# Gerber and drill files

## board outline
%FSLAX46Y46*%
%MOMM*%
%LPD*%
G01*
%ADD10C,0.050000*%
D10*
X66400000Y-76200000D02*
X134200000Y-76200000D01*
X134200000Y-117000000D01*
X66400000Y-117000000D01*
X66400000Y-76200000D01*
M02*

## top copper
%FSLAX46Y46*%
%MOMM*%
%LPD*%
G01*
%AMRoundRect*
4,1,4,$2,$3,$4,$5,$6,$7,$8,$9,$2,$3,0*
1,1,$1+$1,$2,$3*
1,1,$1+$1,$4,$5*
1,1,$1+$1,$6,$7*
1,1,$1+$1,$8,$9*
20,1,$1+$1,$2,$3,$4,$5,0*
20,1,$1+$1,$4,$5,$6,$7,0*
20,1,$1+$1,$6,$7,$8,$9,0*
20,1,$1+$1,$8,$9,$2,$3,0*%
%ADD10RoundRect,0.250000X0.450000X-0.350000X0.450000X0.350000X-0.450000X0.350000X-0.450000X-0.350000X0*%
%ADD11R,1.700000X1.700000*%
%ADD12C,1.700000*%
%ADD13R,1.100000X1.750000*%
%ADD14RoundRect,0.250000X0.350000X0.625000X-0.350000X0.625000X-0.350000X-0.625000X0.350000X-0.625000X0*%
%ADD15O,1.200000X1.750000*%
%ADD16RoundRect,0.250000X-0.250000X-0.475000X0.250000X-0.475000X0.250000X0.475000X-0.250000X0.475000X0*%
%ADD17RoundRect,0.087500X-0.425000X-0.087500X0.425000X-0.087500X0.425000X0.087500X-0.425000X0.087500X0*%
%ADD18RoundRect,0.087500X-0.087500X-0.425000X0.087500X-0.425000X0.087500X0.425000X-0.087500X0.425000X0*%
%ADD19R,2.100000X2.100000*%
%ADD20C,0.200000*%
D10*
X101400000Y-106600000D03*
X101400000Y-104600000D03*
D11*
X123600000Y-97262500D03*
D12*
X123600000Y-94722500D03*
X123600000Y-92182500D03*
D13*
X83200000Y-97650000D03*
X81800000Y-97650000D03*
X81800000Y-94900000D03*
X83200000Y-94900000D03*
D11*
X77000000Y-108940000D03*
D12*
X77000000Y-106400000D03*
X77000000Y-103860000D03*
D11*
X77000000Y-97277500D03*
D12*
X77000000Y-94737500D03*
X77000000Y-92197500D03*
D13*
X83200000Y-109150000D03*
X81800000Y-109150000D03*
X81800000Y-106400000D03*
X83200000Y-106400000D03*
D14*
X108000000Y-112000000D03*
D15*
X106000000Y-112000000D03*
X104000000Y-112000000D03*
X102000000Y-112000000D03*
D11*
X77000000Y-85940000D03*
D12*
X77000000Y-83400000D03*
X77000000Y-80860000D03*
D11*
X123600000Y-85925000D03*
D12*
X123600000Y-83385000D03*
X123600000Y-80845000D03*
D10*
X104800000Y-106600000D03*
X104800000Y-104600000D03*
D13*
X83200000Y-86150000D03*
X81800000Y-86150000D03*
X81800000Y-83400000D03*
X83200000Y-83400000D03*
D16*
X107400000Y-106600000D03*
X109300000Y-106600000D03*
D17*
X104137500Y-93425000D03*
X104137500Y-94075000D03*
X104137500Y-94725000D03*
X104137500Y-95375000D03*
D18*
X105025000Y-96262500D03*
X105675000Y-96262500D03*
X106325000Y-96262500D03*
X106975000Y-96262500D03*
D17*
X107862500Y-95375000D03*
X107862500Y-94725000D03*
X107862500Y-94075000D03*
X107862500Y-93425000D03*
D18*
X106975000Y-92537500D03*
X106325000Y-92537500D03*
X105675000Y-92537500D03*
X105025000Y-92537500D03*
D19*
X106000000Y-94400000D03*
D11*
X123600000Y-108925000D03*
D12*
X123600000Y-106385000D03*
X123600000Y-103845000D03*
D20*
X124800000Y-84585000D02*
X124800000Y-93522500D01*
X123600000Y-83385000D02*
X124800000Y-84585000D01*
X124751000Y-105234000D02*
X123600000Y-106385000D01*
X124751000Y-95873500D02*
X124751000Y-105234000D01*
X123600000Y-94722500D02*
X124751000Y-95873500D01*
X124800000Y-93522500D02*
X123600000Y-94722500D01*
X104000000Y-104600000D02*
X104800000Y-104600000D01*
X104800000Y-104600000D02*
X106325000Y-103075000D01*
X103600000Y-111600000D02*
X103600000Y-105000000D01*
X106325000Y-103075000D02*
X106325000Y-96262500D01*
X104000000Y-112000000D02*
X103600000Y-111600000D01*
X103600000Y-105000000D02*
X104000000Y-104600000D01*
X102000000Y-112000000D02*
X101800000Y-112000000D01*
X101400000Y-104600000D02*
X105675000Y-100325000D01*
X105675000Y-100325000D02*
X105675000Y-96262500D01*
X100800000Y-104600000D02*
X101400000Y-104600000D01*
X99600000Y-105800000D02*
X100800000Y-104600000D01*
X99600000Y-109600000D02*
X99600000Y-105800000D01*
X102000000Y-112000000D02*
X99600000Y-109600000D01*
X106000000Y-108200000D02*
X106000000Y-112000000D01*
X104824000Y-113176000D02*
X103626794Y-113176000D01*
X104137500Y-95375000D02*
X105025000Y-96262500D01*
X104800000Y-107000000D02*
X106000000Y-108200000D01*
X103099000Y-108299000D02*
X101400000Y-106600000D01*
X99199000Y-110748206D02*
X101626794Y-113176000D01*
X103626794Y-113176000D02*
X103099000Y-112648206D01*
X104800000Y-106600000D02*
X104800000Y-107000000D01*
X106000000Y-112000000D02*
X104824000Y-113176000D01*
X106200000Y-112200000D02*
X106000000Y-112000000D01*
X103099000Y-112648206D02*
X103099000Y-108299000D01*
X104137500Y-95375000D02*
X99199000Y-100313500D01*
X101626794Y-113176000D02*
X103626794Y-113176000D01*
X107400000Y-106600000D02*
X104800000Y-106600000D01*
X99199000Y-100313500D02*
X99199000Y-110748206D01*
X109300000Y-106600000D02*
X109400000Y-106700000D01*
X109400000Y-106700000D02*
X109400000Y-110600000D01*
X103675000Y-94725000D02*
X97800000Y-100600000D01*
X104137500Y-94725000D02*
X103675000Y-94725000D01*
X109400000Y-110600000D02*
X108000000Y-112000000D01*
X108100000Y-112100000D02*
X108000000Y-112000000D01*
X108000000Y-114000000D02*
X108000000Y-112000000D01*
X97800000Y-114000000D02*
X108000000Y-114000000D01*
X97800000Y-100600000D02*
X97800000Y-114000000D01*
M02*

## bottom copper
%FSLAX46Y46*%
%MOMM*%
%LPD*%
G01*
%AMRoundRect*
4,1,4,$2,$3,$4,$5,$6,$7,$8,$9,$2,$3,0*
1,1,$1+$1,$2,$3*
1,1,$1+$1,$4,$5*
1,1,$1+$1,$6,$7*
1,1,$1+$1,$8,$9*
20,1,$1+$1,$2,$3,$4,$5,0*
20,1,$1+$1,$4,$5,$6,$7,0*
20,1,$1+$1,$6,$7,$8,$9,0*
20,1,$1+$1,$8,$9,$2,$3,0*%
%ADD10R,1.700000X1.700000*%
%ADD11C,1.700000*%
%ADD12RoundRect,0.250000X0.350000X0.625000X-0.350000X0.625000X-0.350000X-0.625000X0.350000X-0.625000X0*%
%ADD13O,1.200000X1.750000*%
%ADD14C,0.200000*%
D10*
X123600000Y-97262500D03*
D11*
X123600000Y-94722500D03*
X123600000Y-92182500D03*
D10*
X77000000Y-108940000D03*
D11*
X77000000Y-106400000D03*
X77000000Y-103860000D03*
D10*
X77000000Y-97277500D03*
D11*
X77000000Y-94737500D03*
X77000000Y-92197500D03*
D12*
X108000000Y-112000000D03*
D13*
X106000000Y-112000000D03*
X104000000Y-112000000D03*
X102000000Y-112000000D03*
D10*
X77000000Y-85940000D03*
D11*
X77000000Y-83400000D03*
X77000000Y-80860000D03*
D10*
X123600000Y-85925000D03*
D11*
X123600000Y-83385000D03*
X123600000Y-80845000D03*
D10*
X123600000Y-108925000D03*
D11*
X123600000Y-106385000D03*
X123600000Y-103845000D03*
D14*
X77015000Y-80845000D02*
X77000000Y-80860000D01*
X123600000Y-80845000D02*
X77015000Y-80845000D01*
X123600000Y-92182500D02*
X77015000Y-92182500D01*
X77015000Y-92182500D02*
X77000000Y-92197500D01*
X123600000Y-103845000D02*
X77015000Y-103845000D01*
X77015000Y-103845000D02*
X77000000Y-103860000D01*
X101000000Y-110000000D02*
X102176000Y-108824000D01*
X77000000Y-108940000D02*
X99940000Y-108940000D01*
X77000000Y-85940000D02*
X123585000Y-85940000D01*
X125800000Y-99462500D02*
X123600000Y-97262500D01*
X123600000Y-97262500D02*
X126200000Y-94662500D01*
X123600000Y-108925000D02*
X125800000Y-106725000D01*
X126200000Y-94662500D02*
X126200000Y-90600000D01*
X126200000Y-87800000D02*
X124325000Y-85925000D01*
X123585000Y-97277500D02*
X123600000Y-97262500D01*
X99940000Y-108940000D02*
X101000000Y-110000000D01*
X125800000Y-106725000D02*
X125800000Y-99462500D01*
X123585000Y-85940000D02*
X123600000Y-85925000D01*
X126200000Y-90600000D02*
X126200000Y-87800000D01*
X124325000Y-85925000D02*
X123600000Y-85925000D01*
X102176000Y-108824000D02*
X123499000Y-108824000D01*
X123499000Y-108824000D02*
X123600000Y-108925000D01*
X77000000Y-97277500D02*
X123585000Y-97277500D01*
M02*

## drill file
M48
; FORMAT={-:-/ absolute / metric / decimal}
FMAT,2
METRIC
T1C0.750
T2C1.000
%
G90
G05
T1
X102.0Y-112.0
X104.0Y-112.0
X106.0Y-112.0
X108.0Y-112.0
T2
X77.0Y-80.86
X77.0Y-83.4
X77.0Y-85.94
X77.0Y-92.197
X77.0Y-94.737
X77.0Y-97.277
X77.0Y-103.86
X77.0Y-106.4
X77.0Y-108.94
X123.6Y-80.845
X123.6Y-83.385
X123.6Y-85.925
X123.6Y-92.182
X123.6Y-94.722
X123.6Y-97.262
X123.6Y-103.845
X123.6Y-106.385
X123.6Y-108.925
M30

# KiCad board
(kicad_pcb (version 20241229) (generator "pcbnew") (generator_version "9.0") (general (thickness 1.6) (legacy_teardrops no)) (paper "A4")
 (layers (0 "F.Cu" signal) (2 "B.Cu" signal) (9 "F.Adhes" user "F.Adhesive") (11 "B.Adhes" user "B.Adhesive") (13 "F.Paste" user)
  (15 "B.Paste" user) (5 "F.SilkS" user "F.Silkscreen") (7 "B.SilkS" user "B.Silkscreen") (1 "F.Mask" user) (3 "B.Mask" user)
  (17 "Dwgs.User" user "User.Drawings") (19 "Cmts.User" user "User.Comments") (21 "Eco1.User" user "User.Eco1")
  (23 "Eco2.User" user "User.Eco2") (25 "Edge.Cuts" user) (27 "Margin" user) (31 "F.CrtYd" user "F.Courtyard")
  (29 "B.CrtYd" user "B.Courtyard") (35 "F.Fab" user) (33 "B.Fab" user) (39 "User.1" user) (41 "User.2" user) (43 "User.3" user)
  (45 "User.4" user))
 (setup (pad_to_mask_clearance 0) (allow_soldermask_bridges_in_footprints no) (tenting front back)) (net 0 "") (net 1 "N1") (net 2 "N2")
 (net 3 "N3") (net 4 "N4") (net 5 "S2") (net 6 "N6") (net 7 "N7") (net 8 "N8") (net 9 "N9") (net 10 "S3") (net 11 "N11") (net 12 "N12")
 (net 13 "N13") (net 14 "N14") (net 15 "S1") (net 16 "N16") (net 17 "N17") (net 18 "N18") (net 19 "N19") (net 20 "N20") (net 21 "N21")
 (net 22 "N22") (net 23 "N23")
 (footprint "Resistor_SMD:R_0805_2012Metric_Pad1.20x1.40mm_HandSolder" (layer "F.Cu") (at 101.4 105.6 90)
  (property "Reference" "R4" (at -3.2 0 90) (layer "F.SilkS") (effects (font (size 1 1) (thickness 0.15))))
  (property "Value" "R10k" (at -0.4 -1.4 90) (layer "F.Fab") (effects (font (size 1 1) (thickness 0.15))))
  (pad "1" smd roundrect (at -1 0 90) (size 1.2 1.4) (layers "F.Cu" "F.Mask" "F.Paste") (roundrect_rratio 0.208333) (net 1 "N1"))
  (pad "2" smd roundrect (at 1 0 90) (size 1.2 1.4) (layers "F.Cu" "F.Mask" "F.Paste") (roundrect_rratio 0.208333) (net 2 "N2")))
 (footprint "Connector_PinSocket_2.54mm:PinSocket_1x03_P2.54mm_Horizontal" (layer "F.Cu") (at 123.6 97.2625 180)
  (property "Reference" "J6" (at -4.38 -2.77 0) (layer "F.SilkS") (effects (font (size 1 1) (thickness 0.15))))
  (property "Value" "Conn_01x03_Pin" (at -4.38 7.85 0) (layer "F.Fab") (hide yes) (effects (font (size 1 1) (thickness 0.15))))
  (pad "1" thru_hole rect (at 0 0 180) (size 1.7 1.7) (drill 1) (layers "*.Cu" "*.Mask") (remove_unused_layers no) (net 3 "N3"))
  (pad "2" thru_hole circle (at 0 2.54 180) (size 1.7 1.7) (drill 1) (layers "*.Cu" "*.Mask") (remove_unused_layers no) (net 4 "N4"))
  (pad "3" thru_hole circle (at 0 5.08 180) (size 1.7 1.7) (drill 1) (layers "*.Cu" "*.Mask") (remove_unused_layers no) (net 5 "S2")))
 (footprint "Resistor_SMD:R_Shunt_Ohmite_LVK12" (layer "F.Cu") (at 82.5 96.275 180)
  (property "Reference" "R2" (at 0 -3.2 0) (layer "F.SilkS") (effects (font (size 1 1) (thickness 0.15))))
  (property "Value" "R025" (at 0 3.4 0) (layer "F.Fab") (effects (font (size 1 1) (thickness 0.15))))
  (pad "1" smd rect (at -0.7 -1.375 180) (size 1.1 1.75) (layers "F.Cu" "F.Mask" "F.Paste") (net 4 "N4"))
  (pad "2" smd rect (at 0.7 -1.375 180) (size 1.1 1.75) (layers "F.Cu" "F.Mask" "F.Paste") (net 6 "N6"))
  (pad "3" smd rect (at 0.7 1.375 180) (size 1.1 1.75) (layers "F.Cu" "F.Mask" "F.Paste") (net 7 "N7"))
  (pad "4" smd rect (at -0.7 1.375 180) (size 1.1 1.75) (layers "F.Cu" "F.Mask" "F.Paste") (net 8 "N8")))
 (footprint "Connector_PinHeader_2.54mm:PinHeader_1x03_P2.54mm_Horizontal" (layer "F.Cu") (at 77 108.94 180)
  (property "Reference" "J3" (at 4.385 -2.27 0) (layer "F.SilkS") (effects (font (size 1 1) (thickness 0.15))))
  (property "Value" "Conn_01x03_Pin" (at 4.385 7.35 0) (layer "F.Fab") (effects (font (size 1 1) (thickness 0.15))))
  (pad "1" thru_hole rect (at 0 0 180) (size 1.7 1.7) (drill 1) (layers "*.Cu" "*.Mask") (remove_unused_layers no) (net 3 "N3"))
  (pad "2" thru_hole circle (at 0 2.54 180) (size 1.7 1.7) (drill 1) (layers "*.Cu" "*.Mask") (remove_unused_layers no) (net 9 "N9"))
  (pad "3" thru_hole circle (at 0 5.08 180) (size 1.7 1.7) (drill 1) (layers "*.Cu" "*.Mask") (remove_unused_layers no) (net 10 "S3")))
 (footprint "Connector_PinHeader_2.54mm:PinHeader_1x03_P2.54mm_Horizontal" (layer "F.Cu") (at 77 97.2775 180)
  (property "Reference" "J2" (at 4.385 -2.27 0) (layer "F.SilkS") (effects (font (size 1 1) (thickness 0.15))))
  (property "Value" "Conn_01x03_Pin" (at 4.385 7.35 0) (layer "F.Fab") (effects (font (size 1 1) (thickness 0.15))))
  (pad "1" thru_hole rect (at 0 0 180) (size 1.7 1.7) (drill 1) (layers "*.Cu" "*.Mask") (remove_unused_layers no) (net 3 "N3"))
  (pad "2" thru_hole circle (at 0 2.54 180) (size 1.7 1.7) (drill 1) (layers "*.Cu" "*.Mask") (remove_unused_layers no) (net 8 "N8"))
  (pad "3" thru_hole circle (at 0 5.08 180) (size 1.7 1.7) (drill 1) (layers "*.Cu" "*.Mask") (remove_unused_layers no) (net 5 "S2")))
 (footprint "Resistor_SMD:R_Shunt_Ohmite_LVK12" (layer "F.Cu") (at 82.5 107.775 180)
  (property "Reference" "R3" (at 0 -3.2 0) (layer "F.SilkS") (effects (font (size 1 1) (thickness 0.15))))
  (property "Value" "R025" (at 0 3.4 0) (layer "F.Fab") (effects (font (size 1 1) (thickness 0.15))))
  (pad "1" smd rect (at -0.7 -1.375 180) (size 1.1 1.75) (layers "F.Cu" "F.Mask" "F.Paste") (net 4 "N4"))
  (pad "2" smd rect (at 0.7 -1.375 180) (size 1.1 1.75) (layers "F.Cu" "F.Mask" "F.Paste") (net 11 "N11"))
  (pad "3" smd rect (at 0.7 1.375 180) (size 1.1 1.75) (layers "F.Cu" "F.Mask" "F.Paste") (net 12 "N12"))
  (pad "4" smd rect (at -0.7 1.375 180) (size 1.1 1.75) (layers "F.Cu" "F.Mask" "F.Paste") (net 9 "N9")))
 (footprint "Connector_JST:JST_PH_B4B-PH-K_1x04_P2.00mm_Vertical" (layer "F.Cu") (at 108 112 180)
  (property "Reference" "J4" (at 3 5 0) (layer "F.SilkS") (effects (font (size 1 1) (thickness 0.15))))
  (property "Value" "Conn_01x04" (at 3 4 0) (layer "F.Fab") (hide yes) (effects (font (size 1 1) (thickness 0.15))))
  (pad "1" thru_hole roundrect (at 0 0 180) (size 1.2 1.75) (drill 0.75) (layers "*.Cu" "*.Mask") (remove_unused_layers no)
   (roundrect_rratio 0.208333) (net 3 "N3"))
  (pad "2" thru_hole oval (at 2 0 180) (size 1.2 1.75) (drill 0.75) (layers "*.Cu" "*.Mask") (remove_unused_layers no) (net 1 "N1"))
  (pad "3" thru_hole oval (at 4 0 180) (size 1.2 1.75) (drill 0.75) (layers "*.Cu" "*.Mask") (remove_unused_layers no) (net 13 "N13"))
  (pad "4" thru_hole oval (at 6 0 180) (size 1.2 1.75) (drill 0.75) (layers "*.Cu" "*.Mask") (remove_unused_layers no) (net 2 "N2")))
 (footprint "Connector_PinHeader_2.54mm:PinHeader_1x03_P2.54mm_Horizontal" (layer "F.Cu") (at 77 85.94 180)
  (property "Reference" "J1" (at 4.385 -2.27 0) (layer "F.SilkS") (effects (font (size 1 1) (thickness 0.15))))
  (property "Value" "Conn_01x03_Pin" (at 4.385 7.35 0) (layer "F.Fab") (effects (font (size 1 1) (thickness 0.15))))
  (pad "1" thru_hole rect (at 0 0 180) (size 1.7 1.7) (drill 1) (layers "*.Cu" "*.Mask") (remove_unused_layers no) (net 3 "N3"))
  (pad "2" thru_hole circle (at 0 2.54 180) (size 1.7 1.7) (drill 1) (layers "*.Cu" "*.Mask") (remove_unused_layers no) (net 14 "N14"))
  (pad "3" thru_hole circle (at 0 5.08 180) (size 1.7 1.7) (drill 1) (layers "*.Cu" "*.Mask") (remove_unused_layers no) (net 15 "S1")))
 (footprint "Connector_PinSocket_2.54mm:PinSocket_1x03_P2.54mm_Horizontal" (layer "F.Cu") (at 123.6 85.925 180)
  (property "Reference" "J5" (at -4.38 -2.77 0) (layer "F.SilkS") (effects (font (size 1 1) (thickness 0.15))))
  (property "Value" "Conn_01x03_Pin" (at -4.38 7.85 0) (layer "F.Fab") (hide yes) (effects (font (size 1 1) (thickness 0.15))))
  (pad "1" thru_hole rect (at 0 0 180) (size 1.7 1.7) (drill 1) (layers "*.Cu" "*.Mask") (remove_unused_layers no) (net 3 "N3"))
  (pad "2" thru_hole circle (at 0 2.54 180) (size 1.7 1.7) (drill 1) (layers "*.Cu" "*.Mask") (remove_unused_layers no) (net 4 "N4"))
  (pad "3" thru_hole circle (at 0 5.08 180) (size 1.7 1.7) (drill 1) (layers "*.Cu" "*.Mask") (remove_unused_layers no) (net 15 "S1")))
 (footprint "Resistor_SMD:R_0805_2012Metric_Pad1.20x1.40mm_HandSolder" (layer "F.Cu") (at 104.8 105.6 90)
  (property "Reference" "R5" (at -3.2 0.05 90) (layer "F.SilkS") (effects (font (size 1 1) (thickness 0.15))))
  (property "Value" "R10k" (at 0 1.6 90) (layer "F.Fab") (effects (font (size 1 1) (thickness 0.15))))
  (pad "1" smd roundrect (at -1 0 90) (size 1.2 1.4) (layers "F.Cu" "F.Mask" "F.Paste") (roundrect_rratio 0.208333) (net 1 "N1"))
  (pad "2" smd roundrect (at 1 0 90) (size 1.2 1.4) (layers "F.Cu" "F.Mask" "F.Paste") (roundrect_rratio 0.208333) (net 13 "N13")))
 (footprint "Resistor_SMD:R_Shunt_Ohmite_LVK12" (layer "F.Cu") (at 82.5 84.775 180)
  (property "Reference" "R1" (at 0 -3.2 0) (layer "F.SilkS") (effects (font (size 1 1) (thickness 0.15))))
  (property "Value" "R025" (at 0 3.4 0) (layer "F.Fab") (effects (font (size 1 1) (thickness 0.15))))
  (pad "1" smd rect (at -0.7 -1.375 180) (size 1.1 1.75) (layers "F.Cu" "F.Mask" "F.Paste") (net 4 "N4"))
  (pad "2" smd rect (at 0.7 -1.375 180) (size 1.1 1.75) (layers "F.Cu" "F.Mask" "F.Paste") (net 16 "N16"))
  (pad "3" smd rect (at 0.7 1.375 180) (size 1.1 1.75) (layers "F.Cu" "F.Mask" "F.Paste") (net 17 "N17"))
  (pad "4" smd rect (at -0.7 1.375 180) (size 1.1 1.75) (layers "F.Cu" "F.Mask" "F.Paste") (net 14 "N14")))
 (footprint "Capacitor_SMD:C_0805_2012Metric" (layer "F.Cu") (at 108.35 106.6)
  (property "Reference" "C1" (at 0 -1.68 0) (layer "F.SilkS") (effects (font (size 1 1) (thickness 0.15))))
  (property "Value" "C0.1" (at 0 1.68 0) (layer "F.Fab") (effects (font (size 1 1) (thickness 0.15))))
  (pad "1" smd roundrect (at -0.95 0) (size 1 1.45) (layers "F.Cu" "F.Mask" "F.Paste") (roundrect_rratio 0.25) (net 1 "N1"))
  (pad "2" smd roundrect (at 0.95 0) (size 1 1.45) (layers "F.Cu" "F.Mask" "F.Paste") (roundrect_rratio 0.25) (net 3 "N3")))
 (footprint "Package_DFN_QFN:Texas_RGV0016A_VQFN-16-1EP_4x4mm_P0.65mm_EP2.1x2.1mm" (layer "F.Cu") (at 106 94.4)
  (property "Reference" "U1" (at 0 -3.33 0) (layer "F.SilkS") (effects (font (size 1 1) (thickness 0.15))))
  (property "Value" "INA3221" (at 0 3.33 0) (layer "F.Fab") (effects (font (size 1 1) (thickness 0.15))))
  (pad "" smd roundrect (at -0.525 -0.525) (size 0.85 0.85) (layers "F.Paste") (roundrect_rratio 0.25))
  (pad "" smd roundrect (at -0.525 0.525) (size 0.85 0.85) (layers "F.Paste") (roundrect_rratio 0.25))
  (pad "" smd roundrect (at 0.525 -0.525) (size 0.85 0.85) (layers "F.Paste") (roundrect_rratio 0.25))
  (pad "" smd roundrect (at 0.525 0.525) (size 0.85 0.85) (layers "F.Paste") (roundrect_rratio 0.25))
  (pad "1" smd roundrect (at -1.8625 -0.975) (size 1.025 0.35) (layers "F.Cu" "F.Mask" "F.Paste") (roundrect_rratio 0.25) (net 12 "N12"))
  (pad "2" smd roundrect (at -1.8625 -0.325) (size 1.025 0.35) (layers "F.Cu" "F.Mask" "F.Paste") (roundrect_rratio 0.25) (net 11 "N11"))
  (pad "3" smd roundrect (at -1.8625 0.325) (size 1.025 0.35) (layers "F.Cu" "F.Mask" "F.Paste") (roundrect_rratio 0.25) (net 3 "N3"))
  (pad "4" smd roundrect (at -1.8625 0.975) (size 1.025 0.35) (layers "F.Cu" "F.Mask" "F.Paste") (roundrect_rratio 0.25) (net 1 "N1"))
  (pad "5" smd roundrect (at -0.975 1.8625) (size 0.35 1.025) (layers "F.Cu" "F.Mask" "F.Paste") (roundrect_rratio 0.25) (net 1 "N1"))
  (pad "6" smd roundrect (at -0.325 1.8625) (size 0.35 1.025) (layers "F.Cu" "F.Mask" "F.Paste") (roundrect_rratio 0.25) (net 2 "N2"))
  (pad "7" smd roundrect (at 0.325 1.8625) (size 0.35 1.025) (layers "F.Cu" "F.Mask" "F.Paste") (roundrect_rratio 0.25) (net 13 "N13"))
  (pad "8" smd roundrect (at 0.975 1.8625) (size 0.35 1.025) (layers "F.Cu" "F.Mask" "F.Paste") (roundrect_rratio 0.25) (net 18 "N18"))
  (pad "9" smd roundrect (at 1.8625 0.975) (size 1.025 0.35) (layers "F.Cu" "F.Mask" "F.Paste") (roundrect_rratio 0.25) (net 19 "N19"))
  (pad "10" smd roundrect (at 1.8625 0.325) (size 1.025 0.35) (layers "F.Cu" "F.Mask" "F.Paste") (roundrect_rratio 0.25) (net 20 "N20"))
  (pad "11" smd roundrect (at 1.8625 -0.325) (size 1.025 0.35) (layers "F.Cu" "F.Mask" "F.Paste") (roundrect_rratio 0.25) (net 17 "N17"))
  (pad "12" smd roundrect (at 1.8625 -0.975) (size 1.025 0.35) (layers "F.Cu" "F.Mask" "F.Paste") (roundrect_rratio 0.25) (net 16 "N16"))
  (pad "13" smd roundrect (at 0.975 -1.8625) (size 0.35 1.025) (layers "F.Cu" "F.Mask" "F.Paste") (roundrect_rratio 0.25) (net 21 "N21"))
  (pad "14" smd roundrect (at 0.325 -1.8625) (size 0.35 1.025) (layers "F.Cu" "F.Mask" "F.Paste") (roundrect_rratio 0.25) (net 7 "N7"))
  (pad "15" smd roundrect (at -0.325 -1.8625) (size 0.35 1.025) (layers "F.Cu" "F.Mask" "F.Paste") (roundrect_rratio 0.25) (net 6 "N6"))
  (pad "16" smd roundrect (at -0.975 -1.8625) (size 0.35 1.025) (layers "F.Cu" "F.Mask" "F.Paste") (roundrect_rratio 0.25) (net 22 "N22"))
  (pad "17" smd rect (at 0 0) (size 2.1 2.1) (layers "F.Cu" "F.Mask") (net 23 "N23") (zone_connect 2)))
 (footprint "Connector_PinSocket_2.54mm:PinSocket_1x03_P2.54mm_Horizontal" (layer "F.Cu") (at 123.6 108.925 180)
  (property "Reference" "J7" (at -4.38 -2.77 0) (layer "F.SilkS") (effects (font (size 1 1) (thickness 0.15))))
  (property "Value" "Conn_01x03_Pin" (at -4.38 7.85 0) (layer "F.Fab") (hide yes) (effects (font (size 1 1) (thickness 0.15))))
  (pad "1" thru_hole rect (at 0 0 180) (size 1.7 1.7) (drill 1) (layers "*.Cu" "*.Mask") (remove_unused_layers no) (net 3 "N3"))
  (pad "2" thru_hole circle (at 0 2.54 180) (size 1.7 1.7) (drill 1) (layers "*.Cu" "*.Mask") (remove_unused_layers no) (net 4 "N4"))
  (pad "3" thru_hole circle (at 0 5.08 180) (size 1.7 1.7) (drill 1) (layers "*.Cu" "*.Mask") (remove_unused_layers no) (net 10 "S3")))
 (gr_rect (start 66.4 76.2) (end 134.2 117) (stroke (width 0.05) (type default)) (fill no) (layer "Edge.Cuts"))
 (segment (start 124.8 84.585) (end 124.8 93.5225) (width 0.2) (layer "F.Cu") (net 4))
 (segment (start 123.6 83.385) (end 124.8 84.585) (width 0.2) (layer "F.Cu") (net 4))
 (segment (start 124.751 105.234) (end 123.6 106.385) (width 0.2) (layer "F.Cu") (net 4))
 (segment (start 124.751 95.8735) (end 124.751 105.234) (width 0.2) (layer "F.Cu") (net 4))
 (segment (start 123.6 94.7225) (end 124.751 95.8735) (width 0.2) (layer "F.Cu") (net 4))
 (segment (start 124.8 93.5225) (end 123.6 94.7225) (width 0.2) (layer "F.Cu") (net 4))
 (segment (start 77.015 80.845) (end 77 80.86) (width 0.2) (layer "B.Cu") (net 15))
 (segment (start 123.6 80.845) (end 77.015 80.845) (width 0.2) (layer "B.Cu") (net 15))
 (segment (start 123.6 92.1825) (end 77.015 92.1825) (width 0.2) (layer "B.Cu") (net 5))
 (segment (start 77.015 92.1825) (end 77 92.1975) (width 0.2) (layer "B.Cu") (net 5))
 (segment (start 123.6 103.845) (end 77.015 103.845) (width 0.2) (layer "B.Cu") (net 10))
 (segment (start 77.015 103.845) (end 77 103.86) (width 0.2) (layer "B.Cu") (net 10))
 (segment (start 104 104.6) (end 104.8 104.6) (width 0.2) (layer "F.Cu") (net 13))
 (segment (start 104.8 104.6) (end 106.325 103.075) (width 0.2) (layer "F.Cu") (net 13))
 (segment (start 103.6 111.6) (end 103.6 105) (width 0.2) (layer "F.Cu") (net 13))
 (segment (start 106.325 103.075) (end 106.325 96.2625) (width 0.2) (layer "F.Cu") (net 13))
 (segment (start 104 112) (end 103.6 111.6) (width 0.2) (layer "F.Cu") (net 13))
 (segment (start 103.6 105) (end 104 104.6) (width 0.2) (layer "F.Cu") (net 13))
 (segment (start 102 112) (end 101.8 112) (width 0.2) (layer "F.Cu") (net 2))
 (segment (start 101.4 104.6) (end 105.675 100.325) (width 0.2) (layer "F.Cu") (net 2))
 (segment (start 105.675 100.325) (end 105.675 96.2625) (width 0.2) (layer "F.Cu") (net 2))
 (segment (start 100.8 104.6) (end 101.4 104.6) (width 0.2) (layer "F.Cu") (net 2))
 (segment (start 99.6 105.8) (end 100.8 104.6) (width 0.2) (layer "F.Cu") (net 2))
 (segment (start 99.6 109.6) (end 99.6 105.8) (width 0.2) (layer "F.Cu") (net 2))
 (segment (start 102 112) (end 99.6 109.6) (width 0.2) (layer "F.Cu") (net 2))
 (segment (start 106 108.2) (end 106 112) (width 0.2) (layer "F.Cu") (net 1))
 (segment (start 104.824 113.176) (end 103.626794 113.176) (width 0.2) (layer "F.Cu") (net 1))
 (segment (start 104.1375 95.375) (end 105.025 96.2625) (width 0.2) (layer "F.Cu") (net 1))
 (segment (start 104.8 107) (end 106 108.2) (width 0.2) (layer "F.Cu") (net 1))
 (segment (start 103.099 108.299) (end 101.4 106.6) (width 0.2) (layer "F.Cu") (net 1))
 (segment (start 99.199 110.748206) (end 101.626794 113.176) (width 0.2) (layer "F.Cu") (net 1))
 (segment (start 103.626794 113.176) (end 103.099 112.648206) (width 0.2) (layer "F.Cu") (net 1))
 (segment (start 104.8 106.6) (end 104.8 107) (width 0.2) (layer "F.Cu") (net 1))
 (segment (start 106 112) (end 104.824 113.176) (width 0.2) (layer "F.Cu") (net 1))
 (segment (start 106.2 112.2) (end 106 112) (width 0.2) (layer "F.Cu") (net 1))
 (segment (start 103.099 112.648206) (end 103.099 108.299) (width 0.2) (layer "F.Cu") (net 1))
 (segment (start 104.1375 95.375) (end 99.199 100.3135) (width 0.2) (layer "F.Cu") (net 1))
 (segment (start 101.626794 113.176) (end 103.626794 113.176) (width 0.2) (layer "F.Cu") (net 1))
 (segment (start 107.4 106.6) (end 104.8 106.6) (width 0.2) (layer "F.Cu") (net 1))
 (segment (start 99.199 100.3135) (end 99.199 110.748206) (width 0.2) (layer "F.Cu") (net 1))
 (segment (start 109.3 106.6) (end 109.4 106.7) (width 0.2) (layer "F.Cu") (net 3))
 (segment (start 109.4 106.7) (end 109.4 110.6) (width 0.2) (layer "F.Cu") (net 3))
 (segment (start 103.675 94.725) (end 97.8 100.6) (width 0.2) (layer "F.Cu") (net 3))
 (segment (start 104.1375 94.725) (end 103.675 94.725) (width 0.2) (layer "F.Cu") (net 3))
 (segment (start 109.4 110.6) (end 108 112) (width 0.2) (layer "F.Cu") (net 3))
 (segment (start 108.1 112.1) (end 108 112) (width 0.2) (layer "F.Cu") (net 3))
 (segment (start 108 114) (end 108 112) (width 0.2) (layer "F.Cu") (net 3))
 (segment (start 97.8 114) (end 108 114) (width 0.2) (layer "F.Cu") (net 3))
 (segment (start 97.8 100.6) (end 97.8 114) (width 0.2) (layer "F.Cu") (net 3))
 (segment (start 101 110) (end 102.176 108.824) (width 0.2) (layer "B.Cu") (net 3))
 (segment (start 77 108.94) (end 99.94 108.94) (width 0.2) (layer "B.Cu") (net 3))
 (segment (start 77 85.94) (end 123.585 85.94) (width 0.2) (layer "B.Cu") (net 3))
 (segment (start 125.8 99.4625) (end 123.6 97.2625) (width 0.2) (layer "B.Cu") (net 3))
 (segment (start 123.6 97.2625) (end 126.2 94.6625) (width 0.2) (layer "B.Cu") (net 3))
 (segment (start 123.6 108.925) (end 125.8 106.725) (width 0.2) (layer "B.Cu") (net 3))
 (segment (start 126.2 94.6625) (end 126.2 90.6) (width 0.2) (layer "B.Cu") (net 3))
 (segment (start 126.2 87.8) (end 124.325 85.925) (width 0.2) (layer "B.Cu") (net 3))
 (segment (start 123.585 97.2775) (end 123.6 97.2625) (width 0.2) (layer "B.Cu") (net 3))
 (segment (start 99.94 108.94) (end 101 110) (width 0.2) (layer "B.Cu") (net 3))
 (segment (start 125.8 106.725) (end 125.8 99.4625) (width 0.2) (layer "B.Cu") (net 3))
 (segment (start 123.585 85.94) (end 123.6 85.925) (width 0.2) (layer "B.Cu") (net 3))
 (segment (start 126.2 90.6) (end 126.2 87.8) (width 0.2) (layer "B.Cu") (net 3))
 (segment (start 124.325 85.925) (end 123.6 85.925) (width 0.2) (layer "B.Cu") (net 3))
 (segment (start 102.176 108.824) (end 123.499 108.824) (width 0.2) (layer "B.Cu") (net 3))
 (segment (start 123.499 108.824) (end 123.6 108.925) (width 0.2) (layer "B.Cu") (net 3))
 (segment (start 77 97.2775) (end 123.585 97.2775) (width 0.2) (layer "B.Cu") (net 3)))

